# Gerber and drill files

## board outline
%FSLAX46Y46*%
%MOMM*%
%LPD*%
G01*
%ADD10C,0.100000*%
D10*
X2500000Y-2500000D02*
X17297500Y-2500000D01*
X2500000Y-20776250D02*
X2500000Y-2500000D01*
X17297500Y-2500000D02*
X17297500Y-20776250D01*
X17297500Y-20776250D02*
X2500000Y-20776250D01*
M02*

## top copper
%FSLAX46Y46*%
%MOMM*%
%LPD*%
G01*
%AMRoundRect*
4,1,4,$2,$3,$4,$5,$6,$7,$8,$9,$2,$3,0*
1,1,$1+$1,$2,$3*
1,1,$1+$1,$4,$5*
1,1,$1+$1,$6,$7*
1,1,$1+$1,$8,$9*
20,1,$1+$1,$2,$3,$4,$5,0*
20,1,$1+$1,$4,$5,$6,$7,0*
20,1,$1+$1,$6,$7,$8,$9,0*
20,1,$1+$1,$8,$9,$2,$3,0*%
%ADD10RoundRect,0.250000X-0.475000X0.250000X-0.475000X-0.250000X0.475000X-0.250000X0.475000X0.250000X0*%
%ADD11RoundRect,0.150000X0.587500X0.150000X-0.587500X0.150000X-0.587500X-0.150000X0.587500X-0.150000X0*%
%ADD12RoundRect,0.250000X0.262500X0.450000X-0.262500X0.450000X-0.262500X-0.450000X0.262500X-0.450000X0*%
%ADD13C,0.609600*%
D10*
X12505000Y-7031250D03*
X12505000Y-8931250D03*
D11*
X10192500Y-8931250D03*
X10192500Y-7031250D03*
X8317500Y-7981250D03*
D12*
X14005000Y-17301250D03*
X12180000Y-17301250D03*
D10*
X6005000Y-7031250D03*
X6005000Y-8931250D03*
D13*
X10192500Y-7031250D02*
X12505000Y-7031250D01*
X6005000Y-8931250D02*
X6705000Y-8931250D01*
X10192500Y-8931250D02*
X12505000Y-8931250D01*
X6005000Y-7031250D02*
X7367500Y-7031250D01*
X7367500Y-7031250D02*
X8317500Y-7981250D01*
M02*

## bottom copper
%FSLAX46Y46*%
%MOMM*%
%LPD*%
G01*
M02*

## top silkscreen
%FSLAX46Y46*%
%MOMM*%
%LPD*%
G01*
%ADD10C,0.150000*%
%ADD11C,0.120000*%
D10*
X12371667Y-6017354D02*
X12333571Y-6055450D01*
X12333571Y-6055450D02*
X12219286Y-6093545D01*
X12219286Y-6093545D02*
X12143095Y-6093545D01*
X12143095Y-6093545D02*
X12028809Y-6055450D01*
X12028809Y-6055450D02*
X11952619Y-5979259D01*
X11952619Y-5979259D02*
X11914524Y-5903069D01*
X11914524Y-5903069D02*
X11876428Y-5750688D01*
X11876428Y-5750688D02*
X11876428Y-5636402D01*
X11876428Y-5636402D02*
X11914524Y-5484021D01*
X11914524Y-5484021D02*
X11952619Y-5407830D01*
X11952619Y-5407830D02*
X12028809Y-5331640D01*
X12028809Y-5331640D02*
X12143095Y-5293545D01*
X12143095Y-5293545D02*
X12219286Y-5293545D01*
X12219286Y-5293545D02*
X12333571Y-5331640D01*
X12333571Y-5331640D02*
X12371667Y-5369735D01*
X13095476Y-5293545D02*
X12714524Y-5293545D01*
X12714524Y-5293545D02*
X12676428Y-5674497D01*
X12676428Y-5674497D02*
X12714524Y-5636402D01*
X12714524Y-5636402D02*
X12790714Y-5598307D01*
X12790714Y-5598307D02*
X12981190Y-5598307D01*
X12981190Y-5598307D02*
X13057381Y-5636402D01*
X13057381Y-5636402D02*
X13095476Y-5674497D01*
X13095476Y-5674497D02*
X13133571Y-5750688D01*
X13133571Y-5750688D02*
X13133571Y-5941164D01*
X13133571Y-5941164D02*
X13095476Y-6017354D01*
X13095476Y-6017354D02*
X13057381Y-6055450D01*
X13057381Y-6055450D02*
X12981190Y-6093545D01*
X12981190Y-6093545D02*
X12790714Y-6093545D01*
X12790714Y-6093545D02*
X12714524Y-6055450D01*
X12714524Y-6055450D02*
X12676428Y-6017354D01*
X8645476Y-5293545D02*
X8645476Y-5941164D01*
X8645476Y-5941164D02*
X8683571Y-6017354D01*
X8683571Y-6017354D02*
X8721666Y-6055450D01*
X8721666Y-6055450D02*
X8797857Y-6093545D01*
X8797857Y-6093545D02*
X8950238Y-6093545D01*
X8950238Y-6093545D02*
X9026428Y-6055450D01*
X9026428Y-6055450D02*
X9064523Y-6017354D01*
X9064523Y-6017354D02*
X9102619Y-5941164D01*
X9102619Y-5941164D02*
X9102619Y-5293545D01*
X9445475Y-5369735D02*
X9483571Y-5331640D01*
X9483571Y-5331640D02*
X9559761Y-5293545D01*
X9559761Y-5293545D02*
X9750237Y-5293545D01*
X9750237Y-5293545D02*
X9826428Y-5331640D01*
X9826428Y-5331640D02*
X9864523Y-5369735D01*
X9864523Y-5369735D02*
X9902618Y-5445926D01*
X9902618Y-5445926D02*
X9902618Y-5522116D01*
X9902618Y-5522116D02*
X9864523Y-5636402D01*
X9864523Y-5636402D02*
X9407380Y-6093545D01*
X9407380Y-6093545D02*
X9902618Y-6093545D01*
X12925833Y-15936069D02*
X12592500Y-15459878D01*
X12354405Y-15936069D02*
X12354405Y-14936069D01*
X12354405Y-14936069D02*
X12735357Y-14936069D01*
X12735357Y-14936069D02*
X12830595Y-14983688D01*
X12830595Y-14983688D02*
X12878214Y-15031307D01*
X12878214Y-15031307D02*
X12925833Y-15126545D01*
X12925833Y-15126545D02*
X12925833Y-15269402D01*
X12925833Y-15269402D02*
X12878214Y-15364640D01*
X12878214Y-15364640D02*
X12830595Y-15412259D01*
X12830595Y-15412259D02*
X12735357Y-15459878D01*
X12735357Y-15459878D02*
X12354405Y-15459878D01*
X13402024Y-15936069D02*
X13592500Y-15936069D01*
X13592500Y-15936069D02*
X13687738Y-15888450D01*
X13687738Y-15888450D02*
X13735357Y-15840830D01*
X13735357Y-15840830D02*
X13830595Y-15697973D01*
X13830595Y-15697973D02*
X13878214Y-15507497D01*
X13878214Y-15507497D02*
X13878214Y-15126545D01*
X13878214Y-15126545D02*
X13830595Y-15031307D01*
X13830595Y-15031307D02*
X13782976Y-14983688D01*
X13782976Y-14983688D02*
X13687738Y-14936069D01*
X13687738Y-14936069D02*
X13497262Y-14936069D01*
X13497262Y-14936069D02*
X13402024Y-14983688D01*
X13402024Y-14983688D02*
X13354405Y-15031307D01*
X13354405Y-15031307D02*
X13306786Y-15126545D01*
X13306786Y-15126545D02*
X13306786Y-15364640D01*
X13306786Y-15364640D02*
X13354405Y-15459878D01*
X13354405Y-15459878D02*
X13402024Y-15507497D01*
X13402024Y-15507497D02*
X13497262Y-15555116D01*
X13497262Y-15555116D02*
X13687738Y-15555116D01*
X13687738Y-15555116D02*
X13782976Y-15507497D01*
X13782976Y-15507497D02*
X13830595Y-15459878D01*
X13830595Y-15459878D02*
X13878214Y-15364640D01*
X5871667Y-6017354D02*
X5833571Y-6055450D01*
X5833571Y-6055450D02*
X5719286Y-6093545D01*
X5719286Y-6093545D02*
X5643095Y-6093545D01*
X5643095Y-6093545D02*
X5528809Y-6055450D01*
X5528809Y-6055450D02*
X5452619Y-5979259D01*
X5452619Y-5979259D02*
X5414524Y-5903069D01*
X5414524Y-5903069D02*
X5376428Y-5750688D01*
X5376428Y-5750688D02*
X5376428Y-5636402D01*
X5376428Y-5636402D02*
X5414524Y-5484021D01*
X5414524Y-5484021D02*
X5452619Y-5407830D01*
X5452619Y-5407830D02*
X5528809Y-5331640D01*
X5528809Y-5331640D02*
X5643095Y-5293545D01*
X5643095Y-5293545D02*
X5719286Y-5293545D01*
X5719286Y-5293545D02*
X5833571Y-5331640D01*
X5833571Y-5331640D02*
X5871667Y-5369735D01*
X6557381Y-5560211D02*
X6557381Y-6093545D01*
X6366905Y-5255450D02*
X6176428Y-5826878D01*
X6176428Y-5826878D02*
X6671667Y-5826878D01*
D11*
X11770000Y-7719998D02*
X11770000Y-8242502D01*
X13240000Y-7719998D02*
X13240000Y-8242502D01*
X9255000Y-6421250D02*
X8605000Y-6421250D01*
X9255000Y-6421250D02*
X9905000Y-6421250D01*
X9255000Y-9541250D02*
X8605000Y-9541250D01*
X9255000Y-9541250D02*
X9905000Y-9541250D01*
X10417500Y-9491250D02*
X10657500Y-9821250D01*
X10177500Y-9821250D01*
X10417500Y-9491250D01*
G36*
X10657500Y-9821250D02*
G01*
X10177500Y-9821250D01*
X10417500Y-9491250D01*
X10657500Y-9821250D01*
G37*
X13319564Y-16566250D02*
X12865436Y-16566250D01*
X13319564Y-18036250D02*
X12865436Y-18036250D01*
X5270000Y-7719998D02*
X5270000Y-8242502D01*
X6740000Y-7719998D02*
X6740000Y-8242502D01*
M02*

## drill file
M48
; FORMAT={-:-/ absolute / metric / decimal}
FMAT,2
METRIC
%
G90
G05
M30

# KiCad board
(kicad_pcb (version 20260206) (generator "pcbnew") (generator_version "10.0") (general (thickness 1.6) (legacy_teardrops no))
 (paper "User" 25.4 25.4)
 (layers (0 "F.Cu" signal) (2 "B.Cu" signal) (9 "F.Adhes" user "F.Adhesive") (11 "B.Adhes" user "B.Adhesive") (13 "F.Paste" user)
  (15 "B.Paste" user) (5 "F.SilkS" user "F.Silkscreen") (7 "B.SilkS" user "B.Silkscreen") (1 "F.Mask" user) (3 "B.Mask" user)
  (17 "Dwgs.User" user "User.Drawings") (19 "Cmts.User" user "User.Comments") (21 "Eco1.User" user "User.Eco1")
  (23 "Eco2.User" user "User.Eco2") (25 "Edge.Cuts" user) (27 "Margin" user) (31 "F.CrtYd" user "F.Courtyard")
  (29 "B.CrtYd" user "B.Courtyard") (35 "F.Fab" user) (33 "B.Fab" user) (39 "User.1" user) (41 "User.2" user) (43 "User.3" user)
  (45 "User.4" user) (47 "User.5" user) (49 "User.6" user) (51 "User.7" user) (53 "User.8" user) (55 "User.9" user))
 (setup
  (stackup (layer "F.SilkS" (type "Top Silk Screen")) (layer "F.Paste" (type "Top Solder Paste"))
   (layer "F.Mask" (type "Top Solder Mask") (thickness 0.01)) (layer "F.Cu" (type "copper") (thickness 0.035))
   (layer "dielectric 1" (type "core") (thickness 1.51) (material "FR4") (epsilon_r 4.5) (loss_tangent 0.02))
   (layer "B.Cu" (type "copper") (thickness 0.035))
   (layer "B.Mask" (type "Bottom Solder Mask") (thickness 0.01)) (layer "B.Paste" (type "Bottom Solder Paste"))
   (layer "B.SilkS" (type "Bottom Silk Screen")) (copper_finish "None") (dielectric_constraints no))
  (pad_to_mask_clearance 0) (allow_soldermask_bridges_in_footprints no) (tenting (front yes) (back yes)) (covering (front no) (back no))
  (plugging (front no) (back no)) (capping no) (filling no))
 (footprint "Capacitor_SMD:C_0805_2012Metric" (layer "F.Cu") (at 12.505 7.98125 -90)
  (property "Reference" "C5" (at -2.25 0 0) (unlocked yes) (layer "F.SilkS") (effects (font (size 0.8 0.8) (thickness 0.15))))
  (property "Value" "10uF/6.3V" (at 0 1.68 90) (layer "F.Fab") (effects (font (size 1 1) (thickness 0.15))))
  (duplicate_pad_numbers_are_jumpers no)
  (fp_line (start -0.261252 0.735) (end 0.261252 0.735) (stroke (width 0.12) (type solid)) (layer "F.SilkS"))
  (fp_line (start -0.261252 -0.735) (end 0.261252 -0.735) (stroke (width 0.12) (type solid)) (layer "F.SilkS"))
  (pad "1" smd roundrect (at -0.95 0 270) (size 1 1.45) (layers "F.Cu" "F.Mask" "F.Paste") (roundrect_rratio 0.25) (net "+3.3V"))
  (pad "2" smd roundrect (at 0.95 0 270) (size 1 1.45) (layers "F.Cu" "F.Mask" "F.Paste") (roundrect_rratio 0.25) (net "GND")))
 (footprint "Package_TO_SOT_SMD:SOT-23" (layer "F.Cu") (at 9.255 7.98125 180)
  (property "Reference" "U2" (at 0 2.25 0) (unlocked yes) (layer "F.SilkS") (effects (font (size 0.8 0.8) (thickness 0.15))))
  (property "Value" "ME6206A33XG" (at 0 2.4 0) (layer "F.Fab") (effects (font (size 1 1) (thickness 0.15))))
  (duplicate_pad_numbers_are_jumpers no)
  (fp_line (start 0 1.56) (end 0.65 1.56) (stroke (width 0.12) (type solid)) (layer "F.SilkS"))
  (fp_line (start 0 1.56) (end -0.65 1.56) (stroke (width 0.12) (type solid)) (layer "F.SilkS"))
  (fp_line (start 0 -1.56) (end 0.65 -1.56) (stroke (width 0.12) (type solid)) (layer "F.SilkS"))
  (fp_line (start 0 -1.56) (end -0.65 -1.56) (stroke (width 0.12) (type solid)) (layer "F.SilkS"))
  (fp_poly
   (pts (xy -1.1625 -1.51) (xy -1.4025 -1.84) (xy -0.9225 -1.84) (xy -1.1625 -1.51)) (stroke (width 0.12) (type solid)) (fill yes)
   (layer "F.SilkS"))
  (pad "1" smd roundrect (at -0.9375 -0.95 180) (size 1.475 0.6) (layers "F.Cu" "F.Mask" "F.Paste") (roundrect_rratio 0.25) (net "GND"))
  (pad "2" smd roundrect (at -0.9375 0.95 180) (size 1.475 0.6) (layers "F.Cu" "F.Mask" "F.Paste") (roundrect_rratio 0.25) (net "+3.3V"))
  (pad "3" smd roundrect (at 0.9375 0 180) (size 1.475 0.6) (layers "F.Cu" "F.Mask" "F.Paste") (roundrect_rratio 0.25) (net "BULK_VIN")))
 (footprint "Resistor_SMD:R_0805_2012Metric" (layer "F.Cu") (at 13.0925 17.30125 180)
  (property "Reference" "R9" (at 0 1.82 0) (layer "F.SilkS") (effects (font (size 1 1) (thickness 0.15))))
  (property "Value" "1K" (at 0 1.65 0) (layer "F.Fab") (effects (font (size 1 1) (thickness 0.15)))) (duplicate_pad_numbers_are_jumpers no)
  (fp_line (start -0.227064 0.735) (end 0.227064 0.735) (stroke (width 0.12) (type solid)) (layer "F.SilkS"))
  (fp_line (start -0.227064 -0.735) (end 0.227064 -0.735) (stroke (width 0.12) (type solid)) (layer "F.SilkS"))
  (pad "1" smd roundrect (at -0.9125 0 180) (size 1.025 1.4) (layers "F.Cu" "F.Mask" "F.Paste") (roundrect_rratio 0.243902) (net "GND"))
  (pad "2" smd roundrect (at 0.9125 0 180) (size 1.025 1.4) (layers "F.Cu" "F.Mask" "F.Paste") (roundrect_rratio 0.243902) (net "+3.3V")))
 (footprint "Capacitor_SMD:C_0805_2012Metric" (layer "F.Cu") (at 6.005 7.98125 -90)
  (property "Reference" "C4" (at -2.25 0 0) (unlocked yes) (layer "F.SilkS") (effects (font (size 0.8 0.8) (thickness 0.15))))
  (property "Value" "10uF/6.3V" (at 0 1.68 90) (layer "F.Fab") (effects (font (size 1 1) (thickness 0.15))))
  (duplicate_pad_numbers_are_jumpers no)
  (fp_line (start -0.261252 0.735) (end 0.261252 0.735) (stroke (width 0.12) (type solid)) (layer "F.SilkS"))
  (fp_line (start -0.261252 -0.735) (end 0.261252 -0.735) (stroke (width 0.12) (type solid)) (layer "F.SilkS"))
  (pad "1" smd roundrect (at -0.95 0 270) (size 1 1.45) (layers "F.Cu" "F.Mask" "F.Paste") (roundrect_rratio 0.25) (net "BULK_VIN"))
  (pad "2" smd roundrect (at 0.95 0 270) (size 1 1.45) (layers "F.Cu" "F.Mask" "F.Paste") (roundrect_rratio 0.25) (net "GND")))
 (gr_line (start 2.5 2.5) (end 17.2975 2.5) (stroke (width 0.1) (type default)) (layer "Edge.Cuts"))
 (gr_line (start 2.5 20.77625) (end 2.5 2.5) (stroke (width 0.1) (type default)) (layer "Edge.Cuts"))
 (gr_line (start 17.2975 2.5) (end 17.2975 20.77625) (stroke (width 0.1) (type default)) (layer "Edge.Cuts"))
 (gr_line (start 17.2975 20.77625) (end 2.5 20.77625) (stroke (width 0.1) (type default)) (layer "Edge.Cuts"))
 (segment (start 10.1925 7.03125) (end 12.505 7.03125) (width 0.6096) (layer "F.Cu") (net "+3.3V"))
 (segment (start 6.005 8.93125) (end 6.705 8.93125) (width 0.6096) (layer "F.Cu") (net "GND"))
 (segment (start 10.1925 8.93125) (end 12.505 8.93125) (width 0.6096) (layer "F.Cu") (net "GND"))
 (segment (start 6.005 7.03125) (end 7.3675 7.03125) (width 0.6096) (layer "F.Cu") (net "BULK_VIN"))
 (segment (start 7.3675 7.03125) (end 8.3175 7.98125) (width 0.6096) (layer "F.Cu") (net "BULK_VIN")))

